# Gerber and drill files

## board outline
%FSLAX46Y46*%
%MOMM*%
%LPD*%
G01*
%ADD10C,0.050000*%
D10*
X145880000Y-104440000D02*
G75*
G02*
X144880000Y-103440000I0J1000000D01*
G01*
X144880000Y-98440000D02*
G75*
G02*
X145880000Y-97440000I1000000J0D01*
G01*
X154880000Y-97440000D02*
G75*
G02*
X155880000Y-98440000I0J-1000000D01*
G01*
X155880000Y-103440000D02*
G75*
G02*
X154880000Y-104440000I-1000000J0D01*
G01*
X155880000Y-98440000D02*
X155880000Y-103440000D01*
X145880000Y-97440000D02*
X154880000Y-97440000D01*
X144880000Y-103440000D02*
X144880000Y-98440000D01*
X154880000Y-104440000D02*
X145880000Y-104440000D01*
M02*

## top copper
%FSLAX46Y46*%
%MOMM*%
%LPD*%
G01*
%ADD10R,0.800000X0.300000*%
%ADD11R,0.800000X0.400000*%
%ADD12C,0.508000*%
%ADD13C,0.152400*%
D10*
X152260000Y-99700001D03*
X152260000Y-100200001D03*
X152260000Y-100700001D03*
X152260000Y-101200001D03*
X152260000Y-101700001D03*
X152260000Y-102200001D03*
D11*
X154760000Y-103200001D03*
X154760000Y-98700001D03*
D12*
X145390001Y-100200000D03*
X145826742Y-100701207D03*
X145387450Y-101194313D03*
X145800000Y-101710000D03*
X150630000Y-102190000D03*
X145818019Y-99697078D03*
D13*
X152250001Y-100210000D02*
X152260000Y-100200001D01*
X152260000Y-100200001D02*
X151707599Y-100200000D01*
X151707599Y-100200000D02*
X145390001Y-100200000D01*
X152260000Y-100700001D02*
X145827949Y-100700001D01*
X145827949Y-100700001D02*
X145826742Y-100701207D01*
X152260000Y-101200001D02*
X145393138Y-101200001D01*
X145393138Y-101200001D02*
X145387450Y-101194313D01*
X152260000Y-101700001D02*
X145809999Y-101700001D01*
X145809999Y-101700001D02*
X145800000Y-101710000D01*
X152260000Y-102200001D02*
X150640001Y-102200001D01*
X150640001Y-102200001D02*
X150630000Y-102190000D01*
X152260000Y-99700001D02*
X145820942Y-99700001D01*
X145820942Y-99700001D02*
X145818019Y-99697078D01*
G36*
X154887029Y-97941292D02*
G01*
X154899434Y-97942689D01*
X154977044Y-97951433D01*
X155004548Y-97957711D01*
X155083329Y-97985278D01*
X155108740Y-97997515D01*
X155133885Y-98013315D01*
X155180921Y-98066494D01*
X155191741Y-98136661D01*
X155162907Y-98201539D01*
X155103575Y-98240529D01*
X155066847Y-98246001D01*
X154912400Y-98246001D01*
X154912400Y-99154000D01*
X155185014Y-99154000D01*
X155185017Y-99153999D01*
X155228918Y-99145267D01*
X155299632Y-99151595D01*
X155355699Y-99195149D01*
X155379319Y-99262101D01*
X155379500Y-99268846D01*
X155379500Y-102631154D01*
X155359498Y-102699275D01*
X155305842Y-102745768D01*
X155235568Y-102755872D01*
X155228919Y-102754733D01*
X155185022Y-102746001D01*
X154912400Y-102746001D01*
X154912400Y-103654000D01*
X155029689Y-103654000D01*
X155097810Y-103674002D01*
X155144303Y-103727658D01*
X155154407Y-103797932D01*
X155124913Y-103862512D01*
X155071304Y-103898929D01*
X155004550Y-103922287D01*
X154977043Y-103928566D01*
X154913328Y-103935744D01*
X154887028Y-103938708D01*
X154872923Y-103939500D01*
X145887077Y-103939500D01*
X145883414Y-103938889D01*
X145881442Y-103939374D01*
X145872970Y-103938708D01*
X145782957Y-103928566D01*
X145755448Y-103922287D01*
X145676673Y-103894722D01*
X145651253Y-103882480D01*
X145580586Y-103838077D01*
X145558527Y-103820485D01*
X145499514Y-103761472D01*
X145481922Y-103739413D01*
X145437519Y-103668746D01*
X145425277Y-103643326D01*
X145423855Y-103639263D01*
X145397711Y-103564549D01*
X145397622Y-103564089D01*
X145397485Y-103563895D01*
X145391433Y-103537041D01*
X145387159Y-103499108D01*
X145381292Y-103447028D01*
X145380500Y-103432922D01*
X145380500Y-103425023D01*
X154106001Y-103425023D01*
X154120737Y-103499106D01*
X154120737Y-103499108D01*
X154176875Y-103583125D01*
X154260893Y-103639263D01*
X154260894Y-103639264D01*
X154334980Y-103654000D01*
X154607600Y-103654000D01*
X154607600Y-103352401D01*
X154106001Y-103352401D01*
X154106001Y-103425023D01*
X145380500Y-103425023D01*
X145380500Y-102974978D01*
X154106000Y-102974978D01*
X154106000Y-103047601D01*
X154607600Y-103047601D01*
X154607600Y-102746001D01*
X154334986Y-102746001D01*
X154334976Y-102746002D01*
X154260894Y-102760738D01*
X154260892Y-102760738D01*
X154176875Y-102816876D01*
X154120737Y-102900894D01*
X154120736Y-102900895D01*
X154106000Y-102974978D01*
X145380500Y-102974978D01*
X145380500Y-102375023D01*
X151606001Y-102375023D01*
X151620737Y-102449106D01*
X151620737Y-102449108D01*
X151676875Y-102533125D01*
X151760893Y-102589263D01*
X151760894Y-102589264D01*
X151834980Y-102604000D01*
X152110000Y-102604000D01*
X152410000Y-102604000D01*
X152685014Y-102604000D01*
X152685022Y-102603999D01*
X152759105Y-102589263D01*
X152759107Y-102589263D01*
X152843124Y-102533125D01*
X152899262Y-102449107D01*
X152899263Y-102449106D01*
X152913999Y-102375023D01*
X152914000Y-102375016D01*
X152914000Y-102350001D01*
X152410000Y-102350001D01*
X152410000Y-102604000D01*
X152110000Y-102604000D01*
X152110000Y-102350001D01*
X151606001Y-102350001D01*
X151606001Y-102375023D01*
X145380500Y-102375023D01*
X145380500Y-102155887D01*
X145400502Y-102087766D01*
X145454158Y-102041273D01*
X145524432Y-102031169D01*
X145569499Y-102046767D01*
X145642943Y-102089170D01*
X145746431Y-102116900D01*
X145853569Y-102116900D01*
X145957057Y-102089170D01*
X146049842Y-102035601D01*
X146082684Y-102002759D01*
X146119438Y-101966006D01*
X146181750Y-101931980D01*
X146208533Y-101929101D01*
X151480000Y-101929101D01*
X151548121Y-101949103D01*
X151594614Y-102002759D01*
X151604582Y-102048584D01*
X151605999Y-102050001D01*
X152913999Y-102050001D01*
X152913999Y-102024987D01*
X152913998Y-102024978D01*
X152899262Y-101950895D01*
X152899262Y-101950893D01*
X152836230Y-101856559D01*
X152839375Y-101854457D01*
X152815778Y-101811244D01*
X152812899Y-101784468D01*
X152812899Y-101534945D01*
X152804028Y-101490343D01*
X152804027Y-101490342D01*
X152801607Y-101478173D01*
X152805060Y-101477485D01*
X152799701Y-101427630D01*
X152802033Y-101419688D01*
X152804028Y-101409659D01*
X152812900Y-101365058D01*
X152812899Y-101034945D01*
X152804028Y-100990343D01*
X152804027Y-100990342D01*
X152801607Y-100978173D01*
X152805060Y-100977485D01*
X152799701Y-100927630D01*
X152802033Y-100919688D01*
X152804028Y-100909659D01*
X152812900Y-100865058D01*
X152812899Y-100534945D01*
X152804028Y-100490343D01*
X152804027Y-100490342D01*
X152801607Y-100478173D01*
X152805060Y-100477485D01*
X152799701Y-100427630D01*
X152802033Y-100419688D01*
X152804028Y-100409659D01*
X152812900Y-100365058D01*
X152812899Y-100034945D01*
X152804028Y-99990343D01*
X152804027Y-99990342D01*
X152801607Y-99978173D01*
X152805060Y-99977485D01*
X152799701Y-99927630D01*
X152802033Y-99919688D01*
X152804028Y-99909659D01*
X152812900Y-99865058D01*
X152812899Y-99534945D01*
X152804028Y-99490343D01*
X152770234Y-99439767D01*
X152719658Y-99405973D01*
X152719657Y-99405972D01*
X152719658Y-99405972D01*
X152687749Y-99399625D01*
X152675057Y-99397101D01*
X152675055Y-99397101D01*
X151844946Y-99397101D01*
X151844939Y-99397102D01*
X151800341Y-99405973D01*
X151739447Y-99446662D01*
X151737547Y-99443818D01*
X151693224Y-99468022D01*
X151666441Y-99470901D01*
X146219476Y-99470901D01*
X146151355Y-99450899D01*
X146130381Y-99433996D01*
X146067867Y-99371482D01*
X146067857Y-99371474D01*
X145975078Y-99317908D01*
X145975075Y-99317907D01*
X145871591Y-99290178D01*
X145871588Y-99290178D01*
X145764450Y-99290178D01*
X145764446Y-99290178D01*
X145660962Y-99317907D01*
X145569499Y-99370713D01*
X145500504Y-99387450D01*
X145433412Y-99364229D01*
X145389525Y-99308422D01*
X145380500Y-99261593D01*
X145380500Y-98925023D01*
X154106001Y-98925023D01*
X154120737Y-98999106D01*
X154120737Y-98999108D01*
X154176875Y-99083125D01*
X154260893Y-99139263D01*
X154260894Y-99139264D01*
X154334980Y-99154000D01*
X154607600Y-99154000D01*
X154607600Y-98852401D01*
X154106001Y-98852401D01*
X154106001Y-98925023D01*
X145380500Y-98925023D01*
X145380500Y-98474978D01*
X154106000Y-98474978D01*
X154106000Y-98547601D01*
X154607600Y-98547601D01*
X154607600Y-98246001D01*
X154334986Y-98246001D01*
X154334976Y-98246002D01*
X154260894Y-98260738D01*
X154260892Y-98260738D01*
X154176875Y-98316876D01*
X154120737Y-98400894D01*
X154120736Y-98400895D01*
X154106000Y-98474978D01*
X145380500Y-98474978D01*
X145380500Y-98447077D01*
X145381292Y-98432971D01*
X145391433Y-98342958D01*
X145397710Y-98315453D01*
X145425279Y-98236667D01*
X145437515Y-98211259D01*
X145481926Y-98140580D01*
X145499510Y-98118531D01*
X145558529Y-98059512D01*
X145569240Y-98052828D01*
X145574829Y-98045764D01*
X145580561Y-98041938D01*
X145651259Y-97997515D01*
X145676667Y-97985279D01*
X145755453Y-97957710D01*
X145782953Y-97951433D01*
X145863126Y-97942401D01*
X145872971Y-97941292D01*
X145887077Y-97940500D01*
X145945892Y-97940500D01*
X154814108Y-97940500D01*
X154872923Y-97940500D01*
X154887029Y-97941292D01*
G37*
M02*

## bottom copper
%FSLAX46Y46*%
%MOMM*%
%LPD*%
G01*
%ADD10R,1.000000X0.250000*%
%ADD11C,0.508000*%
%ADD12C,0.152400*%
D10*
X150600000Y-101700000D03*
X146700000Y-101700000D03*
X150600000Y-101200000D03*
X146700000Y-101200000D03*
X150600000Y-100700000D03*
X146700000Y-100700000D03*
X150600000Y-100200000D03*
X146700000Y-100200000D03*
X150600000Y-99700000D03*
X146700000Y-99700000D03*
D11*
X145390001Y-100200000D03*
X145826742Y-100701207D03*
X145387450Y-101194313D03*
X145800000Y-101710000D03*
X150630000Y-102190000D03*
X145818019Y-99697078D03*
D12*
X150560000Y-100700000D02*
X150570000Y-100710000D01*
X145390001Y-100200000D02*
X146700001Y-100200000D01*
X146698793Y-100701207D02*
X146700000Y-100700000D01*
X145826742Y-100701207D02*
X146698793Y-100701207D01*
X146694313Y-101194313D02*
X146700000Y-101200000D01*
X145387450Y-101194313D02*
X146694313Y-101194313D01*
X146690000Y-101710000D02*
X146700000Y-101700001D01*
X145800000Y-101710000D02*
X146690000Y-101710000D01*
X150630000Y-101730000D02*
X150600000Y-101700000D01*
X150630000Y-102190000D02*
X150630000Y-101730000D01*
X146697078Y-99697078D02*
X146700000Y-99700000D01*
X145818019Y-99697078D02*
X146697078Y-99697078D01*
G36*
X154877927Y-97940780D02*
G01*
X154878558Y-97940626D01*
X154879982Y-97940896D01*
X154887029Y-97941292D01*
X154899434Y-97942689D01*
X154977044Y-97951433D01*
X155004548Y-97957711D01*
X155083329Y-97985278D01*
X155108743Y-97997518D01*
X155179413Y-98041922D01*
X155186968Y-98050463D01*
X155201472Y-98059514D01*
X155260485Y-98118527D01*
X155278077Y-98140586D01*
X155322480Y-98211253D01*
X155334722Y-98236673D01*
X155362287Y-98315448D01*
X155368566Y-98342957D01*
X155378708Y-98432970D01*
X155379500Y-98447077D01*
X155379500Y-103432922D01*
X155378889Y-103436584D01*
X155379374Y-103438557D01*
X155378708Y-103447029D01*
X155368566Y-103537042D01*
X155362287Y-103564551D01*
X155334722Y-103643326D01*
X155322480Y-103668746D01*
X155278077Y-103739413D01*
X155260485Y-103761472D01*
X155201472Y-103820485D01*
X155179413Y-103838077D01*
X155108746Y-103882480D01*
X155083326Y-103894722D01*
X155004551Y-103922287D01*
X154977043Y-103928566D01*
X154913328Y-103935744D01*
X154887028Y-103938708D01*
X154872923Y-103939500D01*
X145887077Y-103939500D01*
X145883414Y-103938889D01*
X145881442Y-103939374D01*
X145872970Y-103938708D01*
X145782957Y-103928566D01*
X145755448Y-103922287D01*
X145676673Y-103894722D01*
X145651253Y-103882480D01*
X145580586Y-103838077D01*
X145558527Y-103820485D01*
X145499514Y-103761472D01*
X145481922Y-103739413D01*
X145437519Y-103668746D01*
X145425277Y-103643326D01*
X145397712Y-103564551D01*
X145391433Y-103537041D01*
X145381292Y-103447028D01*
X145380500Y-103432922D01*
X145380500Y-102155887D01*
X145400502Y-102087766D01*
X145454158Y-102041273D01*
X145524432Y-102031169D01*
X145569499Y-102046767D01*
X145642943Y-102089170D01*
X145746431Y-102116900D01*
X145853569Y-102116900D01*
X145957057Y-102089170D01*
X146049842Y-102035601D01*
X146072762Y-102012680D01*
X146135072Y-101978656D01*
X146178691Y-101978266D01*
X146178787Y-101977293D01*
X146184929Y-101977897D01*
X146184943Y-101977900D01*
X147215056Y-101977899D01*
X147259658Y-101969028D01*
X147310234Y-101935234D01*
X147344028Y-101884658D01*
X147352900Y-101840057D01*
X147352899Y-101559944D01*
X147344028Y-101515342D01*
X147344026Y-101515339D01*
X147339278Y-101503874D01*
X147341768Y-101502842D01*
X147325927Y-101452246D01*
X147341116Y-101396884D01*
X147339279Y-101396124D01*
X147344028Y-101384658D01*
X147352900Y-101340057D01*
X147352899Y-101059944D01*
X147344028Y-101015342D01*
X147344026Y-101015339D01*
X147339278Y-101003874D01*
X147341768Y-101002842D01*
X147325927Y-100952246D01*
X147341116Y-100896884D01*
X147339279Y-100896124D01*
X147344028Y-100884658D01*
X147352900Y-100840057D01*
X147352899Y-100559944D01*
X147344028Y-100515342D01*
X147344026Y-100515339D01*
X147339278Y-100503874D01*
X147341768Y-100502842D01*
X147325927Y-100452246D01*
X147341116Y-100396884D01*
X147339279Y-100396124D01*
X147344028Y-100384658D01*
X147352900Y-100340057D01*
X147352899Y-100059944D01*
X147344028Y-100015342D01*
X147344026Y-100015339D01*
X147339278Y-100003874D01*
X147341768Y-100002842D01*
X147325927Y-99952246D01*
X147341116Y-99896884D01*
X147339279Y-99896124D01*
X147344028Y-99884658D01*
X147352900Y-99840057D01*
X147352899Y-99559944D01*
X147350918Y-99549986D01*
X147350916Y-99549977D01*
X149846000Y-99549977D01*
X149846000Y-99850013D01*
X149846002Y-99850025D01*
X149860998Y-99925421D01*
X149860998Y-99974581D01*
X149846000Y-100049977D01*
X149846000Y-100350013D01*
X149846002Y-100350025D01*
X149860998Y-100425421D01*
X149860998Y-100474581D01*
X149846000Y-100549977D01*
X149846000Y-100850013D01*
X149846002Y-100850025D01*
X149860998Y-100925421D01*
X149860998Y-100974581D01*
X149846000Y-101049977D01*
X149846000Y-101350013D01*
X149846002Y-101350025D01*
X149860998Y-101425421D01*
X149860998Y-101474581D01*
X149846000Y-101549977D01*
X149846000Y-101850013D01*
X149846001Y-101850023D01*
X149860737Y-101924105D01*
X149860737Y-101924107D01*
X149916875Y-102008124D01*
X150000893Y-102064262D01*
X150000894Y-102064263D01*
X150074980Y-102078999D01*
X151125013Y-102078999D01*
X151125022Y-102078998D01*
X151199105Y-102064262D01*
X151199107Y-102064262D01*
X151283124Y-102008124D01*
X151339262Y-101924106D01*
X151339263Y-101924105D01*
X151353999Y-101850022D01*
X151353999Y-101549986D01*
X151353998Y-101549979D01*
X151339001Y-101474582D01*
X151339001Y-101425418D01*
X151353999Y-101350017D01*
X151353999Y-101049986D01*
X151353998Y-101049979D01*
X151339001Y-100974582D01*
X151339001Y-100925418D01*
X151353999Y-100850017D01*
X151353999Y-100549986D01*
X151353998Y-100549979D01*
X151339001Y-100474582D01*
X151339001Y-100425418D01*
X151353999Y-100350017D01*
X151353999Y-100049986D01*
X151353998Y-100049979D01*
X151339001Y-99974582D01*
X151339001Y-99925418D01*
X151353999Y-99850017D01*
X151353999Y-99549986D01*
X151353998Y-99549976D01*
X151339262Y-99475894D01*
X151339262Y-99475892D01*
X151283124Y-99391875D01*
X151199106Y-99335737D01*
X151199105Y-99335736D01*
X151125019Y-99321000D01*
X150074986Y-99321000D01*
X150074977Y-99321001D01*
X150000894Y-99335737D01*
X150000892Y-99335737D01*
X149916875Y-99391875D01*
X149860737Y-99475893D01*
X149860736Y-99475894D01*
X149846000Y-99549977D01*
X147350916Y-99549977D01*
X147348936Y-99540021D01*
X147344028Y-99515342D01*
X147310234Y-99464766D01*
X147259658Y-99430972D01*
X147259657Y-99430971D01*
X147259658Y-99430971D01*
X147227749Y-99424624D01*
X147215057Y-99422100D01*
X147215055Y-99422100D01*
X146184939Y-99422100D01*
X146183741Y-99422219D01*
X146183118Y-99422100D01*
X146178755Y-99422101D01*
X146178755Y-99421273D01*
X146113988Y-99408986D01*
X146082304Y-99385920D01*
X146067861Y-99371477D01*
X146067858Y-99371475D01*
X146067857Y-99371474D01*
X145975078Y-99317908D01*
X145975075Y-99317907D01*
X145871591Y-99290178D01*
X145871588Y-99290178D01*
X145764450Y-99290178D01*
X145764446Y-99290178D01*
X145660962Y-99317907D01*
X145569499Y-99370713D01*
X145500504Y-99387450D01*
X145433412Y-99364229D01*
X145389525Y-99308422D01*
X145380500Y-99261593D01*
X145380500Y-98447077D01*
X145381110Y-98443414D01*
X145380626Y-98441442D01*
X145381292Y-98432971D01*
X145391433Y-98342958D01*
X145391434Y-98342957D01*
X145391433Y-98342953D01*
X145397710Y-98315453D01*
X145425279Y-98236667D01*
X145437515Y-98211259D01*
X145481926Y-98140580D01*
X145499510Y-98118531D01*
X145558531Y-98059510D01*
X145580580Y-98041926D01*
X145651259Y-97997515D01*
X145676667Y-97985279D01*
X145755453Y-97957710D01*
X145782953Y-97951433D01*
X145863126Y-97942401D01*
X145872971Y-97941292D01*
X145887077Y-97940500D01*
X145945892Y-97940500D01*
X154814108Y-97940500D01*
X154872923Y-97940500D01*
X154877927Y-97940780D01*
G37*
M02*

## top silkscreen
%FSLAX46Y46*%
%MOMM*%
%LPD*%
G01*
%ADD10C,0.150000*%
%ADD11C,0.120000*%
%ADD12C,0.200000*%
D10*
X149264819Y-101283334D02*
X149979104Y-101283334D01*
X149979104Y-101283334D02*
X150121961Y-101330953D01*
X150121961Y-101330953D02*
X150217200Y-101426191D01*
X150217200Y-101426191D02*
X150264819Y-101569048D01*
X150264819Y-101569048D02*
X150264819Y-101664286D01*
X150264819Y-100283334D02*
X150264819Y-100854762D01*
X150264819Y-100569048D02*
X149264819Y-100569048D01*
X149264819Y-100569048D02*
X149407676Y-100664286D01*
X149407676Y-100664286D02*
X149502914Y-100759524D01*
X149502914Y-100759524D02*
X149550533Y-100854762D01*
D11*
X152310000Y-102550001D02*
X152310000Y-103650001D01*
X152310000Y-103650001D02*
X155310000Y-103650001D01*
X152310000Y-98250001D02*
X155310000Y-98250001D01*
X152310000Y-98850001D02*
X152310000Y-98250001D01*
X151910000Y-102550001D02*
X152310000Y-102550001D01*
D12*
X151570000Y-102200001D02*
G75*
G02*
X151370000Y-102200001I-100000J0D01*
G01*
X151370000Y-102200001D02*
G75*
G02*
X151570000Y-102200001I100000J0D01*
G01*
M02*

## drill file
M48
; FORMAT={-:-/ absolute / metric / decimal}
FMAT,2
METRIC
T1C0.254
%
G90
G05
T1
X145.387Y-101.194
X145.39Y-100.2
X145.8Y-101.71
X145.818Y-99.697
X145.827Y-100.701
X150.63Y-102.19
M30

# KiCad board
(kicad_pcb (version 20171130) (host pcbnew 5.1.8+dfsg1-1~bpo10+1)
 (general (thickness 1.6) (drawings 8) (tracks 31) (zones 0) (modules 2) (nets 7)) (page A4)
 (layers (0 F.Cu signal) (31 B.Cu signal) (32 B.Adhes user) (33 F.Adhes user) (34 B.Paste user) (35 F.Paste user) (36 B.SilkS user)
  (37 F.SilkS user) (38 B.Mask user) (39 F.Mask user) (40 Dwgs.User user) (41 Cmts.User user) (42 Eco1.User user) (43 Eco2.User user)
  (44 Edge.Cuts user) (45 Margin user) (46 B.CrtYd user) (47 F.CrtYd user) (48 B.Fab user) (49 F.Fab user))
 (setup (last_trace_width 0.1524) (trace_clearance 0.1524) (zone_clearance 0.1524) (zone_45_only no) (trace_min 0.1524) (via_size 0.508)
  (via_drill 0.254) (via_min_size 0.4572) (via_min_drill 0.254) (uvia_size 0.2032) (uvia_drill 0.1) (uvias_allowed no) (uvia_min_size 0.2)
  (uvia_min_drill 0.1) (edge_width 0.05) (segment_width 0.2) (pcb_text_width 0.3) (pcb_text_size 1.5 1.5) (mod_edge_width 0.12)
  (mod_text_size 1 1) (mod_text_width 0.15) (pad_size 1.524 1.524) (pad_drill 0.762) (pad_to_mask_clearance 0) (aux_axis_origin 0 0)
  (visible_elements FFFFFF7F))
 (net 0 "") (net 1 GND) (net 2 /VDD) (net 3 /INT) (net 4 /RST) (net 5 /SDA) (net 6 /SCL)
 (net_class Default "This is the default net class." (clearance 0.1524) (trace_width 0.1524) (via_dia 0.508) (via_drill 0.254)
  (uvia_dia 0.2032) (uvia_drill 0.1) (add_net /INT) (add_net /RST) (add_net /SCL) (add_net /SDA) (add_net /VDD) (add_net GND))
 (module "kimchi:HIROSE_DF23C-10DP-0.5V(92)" (layer B.Cu) (at 148.65 100.7 270)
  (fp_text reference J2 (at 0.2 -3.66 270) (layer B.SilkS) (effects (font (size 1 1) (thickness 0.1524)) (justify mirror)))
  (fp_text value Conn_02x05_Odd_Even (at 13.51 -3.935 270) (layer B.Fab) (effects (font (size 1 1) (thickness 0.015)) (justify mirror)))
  (pad 10 smd rect (at 1 -1.95 270) (size 0.25 1) (layers B.Cu B.Paste B.Mask) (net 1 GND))
  (pad 9 smd rect (at 1 1.95 270) (size 0.25 1) (layers B.Cu B.Paste B.Mask) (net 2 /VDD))
  (pad 8 smd rect (at 0.5 -1.95 270) (size 0.25 1) (layers B.Cu B.Paste B.Mask) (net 1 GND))
  (pad 7 smd rect (at 0.5 1.95 270) (size 0.25 1) (layers B.Cu B.Paste B.Mask) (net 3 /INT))
  (pad 6 smd rect (at 0 -1.95 270) (size 0.25 1) (layers B.Cu B.Paste B.Mask) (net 1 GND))
  (pad 5 smd rect (at 0 1.95 270) (size 0.25 1) (layers B.Cu B.Paste B.Mask) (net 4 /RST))
  (pad 4 smd rect (at -0.5 -1.95 270) (size 0.25 1) (layers B.Cu B.Paste B.Mask) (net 1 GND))
  (pad 3 smd rect (at -0.5 1.95 270) (size 0.25 1) (layers B.Cu B.Paste B.Mask) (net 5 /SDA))
  (pad 2 smd rect (at -1 -1.95 270) (size 0.25 1) (layers B.Cu B.Paste B.Mask) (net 1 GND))
  (pad 1 smd rect (at -1 1.95 270) (size 0.25 1) (layers B.Cu B.Paste B.Mask) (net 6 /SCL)))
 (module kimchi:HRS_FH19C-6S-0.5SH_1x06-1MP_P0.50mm (layer F.Cu) (at 153.51 100.950001 90)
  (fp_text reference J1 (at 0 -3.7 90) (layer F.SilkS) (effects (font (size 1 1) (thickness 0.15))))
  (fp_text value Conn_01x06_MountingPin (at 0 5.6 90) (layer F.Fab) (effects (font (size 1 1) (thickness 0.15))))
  (fp_line (start -1.6 -1.2) (end -2.7 -1.2) (layer F.SilkS) (width 0.12))
  (fp_line (start -2.7 -1.2) (end -2.7 1.8) (layer F.SilkS) (width 0.12))
  (fp_line (start 2.7 -1.2) (end 2.7 1.8) (layer F.SilkS) (width 0.12))
  (fp_line (start 2.1 -1.2) (end 2.7 -1.2) (layer F.SilkS) (width 0.12))
  (fp_line (start -1.6 -1.6) (end -1.6 -1.2) (layer F.SilkS) (width 0.12))
  (fp_circle (center -1.25 -2.04) (end -1.15 -2.04) (layer F.SilkS) (width 0.2))
  (pad 6 smd rect (at 1.25 -1.25 90) (size 0.3 0.8) (layers F.Cu F.Paste F.Mask) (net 6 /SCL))
  (pad 5 smd rect (at 0.75 -1.25 90) (size 0.3 0.8) (layers F.Cu F.Paste F.Mask) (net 5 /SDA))
  (pad 4 smd rect (at 0.25 -1.25 90) (size 0.3 0.8) (layers F.Cu F.Paste F.Mask) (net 4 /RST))
  (pad 3 smd rect (at -0.25 -1.25 90) (size 0.3 0.8) (layers F.Cu F.Paste F.Mask) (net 3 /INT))
  (pad 2 smd rect (at -0.75 -1.25 90) (size 0.3 0.8) (layers F.Cu F.Paste F.Mask) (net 2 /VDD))
  (pad 1 smd rect (at -1.25 -1.25 90) (size 0.3 0.8) (layers F.Cu F.Paste F.Mask) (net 1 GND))
  (pad MP smd rect (at -2.25 1.25 90) (size 0.4 0.8) (layers F.Cu F.Paste F.Mask) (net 1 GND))
  (pad MP smd rect (at 2.25 1.25 90) (size 0.4 0.8) (layers F.Cu F.Paste F.Mask) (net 1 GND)))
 (gr_arc (start 145.88 103.44) (end 144.88 103.44) (angle -90) (layer Edge.Cuts) (width 0.05))
 (gr_arc (start 145.88 98.44) (end 145.88 97.44) (angle -90) (layer Edge.Cuts) (width 0.05))
 (gr_arc (start 154.88 98.44) (end 155.88 98.44) (angle -90) (layer Edge.Cuts) (width 0.05))
 (gr_arc (start 154.88 103.44) (end 154.88 104.44) (angle -90) (layer Edge.Cuts) (width 0.05))
 (gr_line (start 155.88 98.44) (end 155.88 103.44) (layer Edge.Cuts) (width 0.05))
 (gr_line (start 145.88 97.44) (end 154.88 97.44) (layer Edge.Cuts) (width 0.05))
 (gr_line (start 144.88 103.44) (end 144.88 98.44) (layer Edge.Cuts) (width 0.05))
 (gr_line (start 154.88 104.44) (end 145.88 104.44) (layer Edge.Cuts) (width 0.05))
 (segment (start 152.250001 100.21) (end 152.26 100.200001) (width 0.1524) (layer F.Cu) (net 5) (status 30))
 (segment (start 150.56 100.7) (end 150.57 100.71) (width 0.1524) (layer B.Cu) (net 1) (status 30))
 (via (at 145.390001 100.2) (size 0.508) (drill 0.254) (layers F.Cu B.Cu) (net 5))
 (segment (start 152.26 100.200001) (end 151.707599 100.2) (width 0.1524) (layer F.Cu) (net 5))
 (segment (start 151.707599 100.2) (end 145.390001 100.2) (width 0.1524) (layer F.Cu) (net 5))
 (segment (start 145.390001 100.2) (end 146.700001 100.2) (width 0.1524) (layer B.Cu) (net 5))
 (via (at 145.826742 100.701207) (size 0.508) (drill 0.254) (layers F.Cu B.Cu) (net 4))
 (segment (start 152.26 100.700001) (end 145.827949 100.700001) (width 0.1524) (layer F.Cu) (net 4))
 (segment (start 145.827949 100.700001) (end 145.826742 100.701207) (width 0.1524) (layer F.Cu) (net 4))
 (segment (start 146.698793 100.701207) (end 146.7 100.7) (width 0.1524) (layer B.Cu) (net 4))
 (segment (start 145.826742 100.701207) (end 146.698793 100.701207) (width 0.1524) (layer B.Cu) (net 4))
 (via (at 145.38745 101.194313) (size 0.508) (drill 0.254) (layers F.Cu B.Cu) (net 3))
 (segment (start 152.26 101.200001) (end 145.393138 101.200001) (width 0.1524) (layer F.Cu) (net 3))
 (segment (start 145.393138 101.200001) (end 145.38745 101.194313) (width 0.1524) (layer F.Cu) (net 3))
 (segment (start 146.694313 101.194313) (end 146.7 101.2) (width 0.1524) (layer B.Cu) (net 3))
 (segment (start 145.38745 101.194313) (end 146.694313 101.194313) (width 0.1524) (layer B.Cu) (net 3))
 (via (at 145.8 101.71) (size 0.508) (drill 0.254) (layers F.Cu B.Cu) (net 2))
 (segment (start 152.26 101.700001) (end 145.809999 101.700001) (width 0.1524) (layer F.Cu) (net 2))
 (segment (start 145.809999 101.700001) (end 145.8 101.71) (width 0.1524) (layer F.Cu) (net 2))
 (segment (start 146.69 101.71) (end 146.7 101.700001) (width 0.1524) (layer B.Cu) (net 2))
 (segment (start 145.8 101.71) (end 146.69 101.71) (width 0.1524) (layer B.Cu) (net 2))
 (via (at 150.63 102.19) (size 0.508) (drill 0.254) (layers F.Cu B.Cu) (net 1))
 (segment (start 152.26 102.200001) (end 150.640001 102.200001) (width 0.1524) (layer F.Cu) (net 1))
 (segment (start 150.640001 102.200001) (end 150.63 102.19) (width 0.1524) (layer F.Cu) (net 1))
 (segment (start 150.63 101.73) (end 150.6 101.7) (width 0.1524) (layer B.Cu) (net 1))
 (segment (start 150.63 102.19) (end 150.63 101.73) (width 0.1524) (layer B.Cu) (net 1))
 (via (at 145.818019 99.697078) (size 0.508) (drill 0.254) (layers F.Cu B.Cu) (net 6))
 (segment (start 152.26 99.700001) (end 145.820942 99.700001) (width 0.1524) (layer F.Cu) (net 6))
 (segment (start 145.820942 99.700001) (end 145.818019 99.697078) (width 0.1524) (layer F.Cu) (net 6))
 (segment (start 146.697078 99.697078) (end 146.7 99.7) (width 0.1524) (layer B.Cu) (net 6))
 (segment (start 145.818019 99.697078) (end 146.697078 99.697078) (width 0.1524) (layer B.Cu) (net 6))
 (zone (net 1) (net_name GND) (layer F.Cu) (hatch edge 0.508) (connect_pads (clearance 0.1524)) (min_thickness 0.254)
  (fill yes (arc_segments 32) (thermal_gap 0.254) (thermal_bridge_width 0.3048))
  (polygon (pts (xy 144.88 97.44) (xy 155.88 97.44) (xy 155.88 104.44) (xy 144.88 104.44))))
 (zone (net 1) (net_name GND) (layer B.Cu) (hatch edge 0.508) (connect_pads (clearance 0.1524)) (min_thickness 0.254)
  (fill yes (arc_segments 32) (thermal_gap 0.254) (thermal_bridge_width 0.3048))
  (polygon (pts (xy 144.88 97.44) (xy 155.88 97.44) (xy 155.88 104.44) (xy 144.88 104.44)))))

